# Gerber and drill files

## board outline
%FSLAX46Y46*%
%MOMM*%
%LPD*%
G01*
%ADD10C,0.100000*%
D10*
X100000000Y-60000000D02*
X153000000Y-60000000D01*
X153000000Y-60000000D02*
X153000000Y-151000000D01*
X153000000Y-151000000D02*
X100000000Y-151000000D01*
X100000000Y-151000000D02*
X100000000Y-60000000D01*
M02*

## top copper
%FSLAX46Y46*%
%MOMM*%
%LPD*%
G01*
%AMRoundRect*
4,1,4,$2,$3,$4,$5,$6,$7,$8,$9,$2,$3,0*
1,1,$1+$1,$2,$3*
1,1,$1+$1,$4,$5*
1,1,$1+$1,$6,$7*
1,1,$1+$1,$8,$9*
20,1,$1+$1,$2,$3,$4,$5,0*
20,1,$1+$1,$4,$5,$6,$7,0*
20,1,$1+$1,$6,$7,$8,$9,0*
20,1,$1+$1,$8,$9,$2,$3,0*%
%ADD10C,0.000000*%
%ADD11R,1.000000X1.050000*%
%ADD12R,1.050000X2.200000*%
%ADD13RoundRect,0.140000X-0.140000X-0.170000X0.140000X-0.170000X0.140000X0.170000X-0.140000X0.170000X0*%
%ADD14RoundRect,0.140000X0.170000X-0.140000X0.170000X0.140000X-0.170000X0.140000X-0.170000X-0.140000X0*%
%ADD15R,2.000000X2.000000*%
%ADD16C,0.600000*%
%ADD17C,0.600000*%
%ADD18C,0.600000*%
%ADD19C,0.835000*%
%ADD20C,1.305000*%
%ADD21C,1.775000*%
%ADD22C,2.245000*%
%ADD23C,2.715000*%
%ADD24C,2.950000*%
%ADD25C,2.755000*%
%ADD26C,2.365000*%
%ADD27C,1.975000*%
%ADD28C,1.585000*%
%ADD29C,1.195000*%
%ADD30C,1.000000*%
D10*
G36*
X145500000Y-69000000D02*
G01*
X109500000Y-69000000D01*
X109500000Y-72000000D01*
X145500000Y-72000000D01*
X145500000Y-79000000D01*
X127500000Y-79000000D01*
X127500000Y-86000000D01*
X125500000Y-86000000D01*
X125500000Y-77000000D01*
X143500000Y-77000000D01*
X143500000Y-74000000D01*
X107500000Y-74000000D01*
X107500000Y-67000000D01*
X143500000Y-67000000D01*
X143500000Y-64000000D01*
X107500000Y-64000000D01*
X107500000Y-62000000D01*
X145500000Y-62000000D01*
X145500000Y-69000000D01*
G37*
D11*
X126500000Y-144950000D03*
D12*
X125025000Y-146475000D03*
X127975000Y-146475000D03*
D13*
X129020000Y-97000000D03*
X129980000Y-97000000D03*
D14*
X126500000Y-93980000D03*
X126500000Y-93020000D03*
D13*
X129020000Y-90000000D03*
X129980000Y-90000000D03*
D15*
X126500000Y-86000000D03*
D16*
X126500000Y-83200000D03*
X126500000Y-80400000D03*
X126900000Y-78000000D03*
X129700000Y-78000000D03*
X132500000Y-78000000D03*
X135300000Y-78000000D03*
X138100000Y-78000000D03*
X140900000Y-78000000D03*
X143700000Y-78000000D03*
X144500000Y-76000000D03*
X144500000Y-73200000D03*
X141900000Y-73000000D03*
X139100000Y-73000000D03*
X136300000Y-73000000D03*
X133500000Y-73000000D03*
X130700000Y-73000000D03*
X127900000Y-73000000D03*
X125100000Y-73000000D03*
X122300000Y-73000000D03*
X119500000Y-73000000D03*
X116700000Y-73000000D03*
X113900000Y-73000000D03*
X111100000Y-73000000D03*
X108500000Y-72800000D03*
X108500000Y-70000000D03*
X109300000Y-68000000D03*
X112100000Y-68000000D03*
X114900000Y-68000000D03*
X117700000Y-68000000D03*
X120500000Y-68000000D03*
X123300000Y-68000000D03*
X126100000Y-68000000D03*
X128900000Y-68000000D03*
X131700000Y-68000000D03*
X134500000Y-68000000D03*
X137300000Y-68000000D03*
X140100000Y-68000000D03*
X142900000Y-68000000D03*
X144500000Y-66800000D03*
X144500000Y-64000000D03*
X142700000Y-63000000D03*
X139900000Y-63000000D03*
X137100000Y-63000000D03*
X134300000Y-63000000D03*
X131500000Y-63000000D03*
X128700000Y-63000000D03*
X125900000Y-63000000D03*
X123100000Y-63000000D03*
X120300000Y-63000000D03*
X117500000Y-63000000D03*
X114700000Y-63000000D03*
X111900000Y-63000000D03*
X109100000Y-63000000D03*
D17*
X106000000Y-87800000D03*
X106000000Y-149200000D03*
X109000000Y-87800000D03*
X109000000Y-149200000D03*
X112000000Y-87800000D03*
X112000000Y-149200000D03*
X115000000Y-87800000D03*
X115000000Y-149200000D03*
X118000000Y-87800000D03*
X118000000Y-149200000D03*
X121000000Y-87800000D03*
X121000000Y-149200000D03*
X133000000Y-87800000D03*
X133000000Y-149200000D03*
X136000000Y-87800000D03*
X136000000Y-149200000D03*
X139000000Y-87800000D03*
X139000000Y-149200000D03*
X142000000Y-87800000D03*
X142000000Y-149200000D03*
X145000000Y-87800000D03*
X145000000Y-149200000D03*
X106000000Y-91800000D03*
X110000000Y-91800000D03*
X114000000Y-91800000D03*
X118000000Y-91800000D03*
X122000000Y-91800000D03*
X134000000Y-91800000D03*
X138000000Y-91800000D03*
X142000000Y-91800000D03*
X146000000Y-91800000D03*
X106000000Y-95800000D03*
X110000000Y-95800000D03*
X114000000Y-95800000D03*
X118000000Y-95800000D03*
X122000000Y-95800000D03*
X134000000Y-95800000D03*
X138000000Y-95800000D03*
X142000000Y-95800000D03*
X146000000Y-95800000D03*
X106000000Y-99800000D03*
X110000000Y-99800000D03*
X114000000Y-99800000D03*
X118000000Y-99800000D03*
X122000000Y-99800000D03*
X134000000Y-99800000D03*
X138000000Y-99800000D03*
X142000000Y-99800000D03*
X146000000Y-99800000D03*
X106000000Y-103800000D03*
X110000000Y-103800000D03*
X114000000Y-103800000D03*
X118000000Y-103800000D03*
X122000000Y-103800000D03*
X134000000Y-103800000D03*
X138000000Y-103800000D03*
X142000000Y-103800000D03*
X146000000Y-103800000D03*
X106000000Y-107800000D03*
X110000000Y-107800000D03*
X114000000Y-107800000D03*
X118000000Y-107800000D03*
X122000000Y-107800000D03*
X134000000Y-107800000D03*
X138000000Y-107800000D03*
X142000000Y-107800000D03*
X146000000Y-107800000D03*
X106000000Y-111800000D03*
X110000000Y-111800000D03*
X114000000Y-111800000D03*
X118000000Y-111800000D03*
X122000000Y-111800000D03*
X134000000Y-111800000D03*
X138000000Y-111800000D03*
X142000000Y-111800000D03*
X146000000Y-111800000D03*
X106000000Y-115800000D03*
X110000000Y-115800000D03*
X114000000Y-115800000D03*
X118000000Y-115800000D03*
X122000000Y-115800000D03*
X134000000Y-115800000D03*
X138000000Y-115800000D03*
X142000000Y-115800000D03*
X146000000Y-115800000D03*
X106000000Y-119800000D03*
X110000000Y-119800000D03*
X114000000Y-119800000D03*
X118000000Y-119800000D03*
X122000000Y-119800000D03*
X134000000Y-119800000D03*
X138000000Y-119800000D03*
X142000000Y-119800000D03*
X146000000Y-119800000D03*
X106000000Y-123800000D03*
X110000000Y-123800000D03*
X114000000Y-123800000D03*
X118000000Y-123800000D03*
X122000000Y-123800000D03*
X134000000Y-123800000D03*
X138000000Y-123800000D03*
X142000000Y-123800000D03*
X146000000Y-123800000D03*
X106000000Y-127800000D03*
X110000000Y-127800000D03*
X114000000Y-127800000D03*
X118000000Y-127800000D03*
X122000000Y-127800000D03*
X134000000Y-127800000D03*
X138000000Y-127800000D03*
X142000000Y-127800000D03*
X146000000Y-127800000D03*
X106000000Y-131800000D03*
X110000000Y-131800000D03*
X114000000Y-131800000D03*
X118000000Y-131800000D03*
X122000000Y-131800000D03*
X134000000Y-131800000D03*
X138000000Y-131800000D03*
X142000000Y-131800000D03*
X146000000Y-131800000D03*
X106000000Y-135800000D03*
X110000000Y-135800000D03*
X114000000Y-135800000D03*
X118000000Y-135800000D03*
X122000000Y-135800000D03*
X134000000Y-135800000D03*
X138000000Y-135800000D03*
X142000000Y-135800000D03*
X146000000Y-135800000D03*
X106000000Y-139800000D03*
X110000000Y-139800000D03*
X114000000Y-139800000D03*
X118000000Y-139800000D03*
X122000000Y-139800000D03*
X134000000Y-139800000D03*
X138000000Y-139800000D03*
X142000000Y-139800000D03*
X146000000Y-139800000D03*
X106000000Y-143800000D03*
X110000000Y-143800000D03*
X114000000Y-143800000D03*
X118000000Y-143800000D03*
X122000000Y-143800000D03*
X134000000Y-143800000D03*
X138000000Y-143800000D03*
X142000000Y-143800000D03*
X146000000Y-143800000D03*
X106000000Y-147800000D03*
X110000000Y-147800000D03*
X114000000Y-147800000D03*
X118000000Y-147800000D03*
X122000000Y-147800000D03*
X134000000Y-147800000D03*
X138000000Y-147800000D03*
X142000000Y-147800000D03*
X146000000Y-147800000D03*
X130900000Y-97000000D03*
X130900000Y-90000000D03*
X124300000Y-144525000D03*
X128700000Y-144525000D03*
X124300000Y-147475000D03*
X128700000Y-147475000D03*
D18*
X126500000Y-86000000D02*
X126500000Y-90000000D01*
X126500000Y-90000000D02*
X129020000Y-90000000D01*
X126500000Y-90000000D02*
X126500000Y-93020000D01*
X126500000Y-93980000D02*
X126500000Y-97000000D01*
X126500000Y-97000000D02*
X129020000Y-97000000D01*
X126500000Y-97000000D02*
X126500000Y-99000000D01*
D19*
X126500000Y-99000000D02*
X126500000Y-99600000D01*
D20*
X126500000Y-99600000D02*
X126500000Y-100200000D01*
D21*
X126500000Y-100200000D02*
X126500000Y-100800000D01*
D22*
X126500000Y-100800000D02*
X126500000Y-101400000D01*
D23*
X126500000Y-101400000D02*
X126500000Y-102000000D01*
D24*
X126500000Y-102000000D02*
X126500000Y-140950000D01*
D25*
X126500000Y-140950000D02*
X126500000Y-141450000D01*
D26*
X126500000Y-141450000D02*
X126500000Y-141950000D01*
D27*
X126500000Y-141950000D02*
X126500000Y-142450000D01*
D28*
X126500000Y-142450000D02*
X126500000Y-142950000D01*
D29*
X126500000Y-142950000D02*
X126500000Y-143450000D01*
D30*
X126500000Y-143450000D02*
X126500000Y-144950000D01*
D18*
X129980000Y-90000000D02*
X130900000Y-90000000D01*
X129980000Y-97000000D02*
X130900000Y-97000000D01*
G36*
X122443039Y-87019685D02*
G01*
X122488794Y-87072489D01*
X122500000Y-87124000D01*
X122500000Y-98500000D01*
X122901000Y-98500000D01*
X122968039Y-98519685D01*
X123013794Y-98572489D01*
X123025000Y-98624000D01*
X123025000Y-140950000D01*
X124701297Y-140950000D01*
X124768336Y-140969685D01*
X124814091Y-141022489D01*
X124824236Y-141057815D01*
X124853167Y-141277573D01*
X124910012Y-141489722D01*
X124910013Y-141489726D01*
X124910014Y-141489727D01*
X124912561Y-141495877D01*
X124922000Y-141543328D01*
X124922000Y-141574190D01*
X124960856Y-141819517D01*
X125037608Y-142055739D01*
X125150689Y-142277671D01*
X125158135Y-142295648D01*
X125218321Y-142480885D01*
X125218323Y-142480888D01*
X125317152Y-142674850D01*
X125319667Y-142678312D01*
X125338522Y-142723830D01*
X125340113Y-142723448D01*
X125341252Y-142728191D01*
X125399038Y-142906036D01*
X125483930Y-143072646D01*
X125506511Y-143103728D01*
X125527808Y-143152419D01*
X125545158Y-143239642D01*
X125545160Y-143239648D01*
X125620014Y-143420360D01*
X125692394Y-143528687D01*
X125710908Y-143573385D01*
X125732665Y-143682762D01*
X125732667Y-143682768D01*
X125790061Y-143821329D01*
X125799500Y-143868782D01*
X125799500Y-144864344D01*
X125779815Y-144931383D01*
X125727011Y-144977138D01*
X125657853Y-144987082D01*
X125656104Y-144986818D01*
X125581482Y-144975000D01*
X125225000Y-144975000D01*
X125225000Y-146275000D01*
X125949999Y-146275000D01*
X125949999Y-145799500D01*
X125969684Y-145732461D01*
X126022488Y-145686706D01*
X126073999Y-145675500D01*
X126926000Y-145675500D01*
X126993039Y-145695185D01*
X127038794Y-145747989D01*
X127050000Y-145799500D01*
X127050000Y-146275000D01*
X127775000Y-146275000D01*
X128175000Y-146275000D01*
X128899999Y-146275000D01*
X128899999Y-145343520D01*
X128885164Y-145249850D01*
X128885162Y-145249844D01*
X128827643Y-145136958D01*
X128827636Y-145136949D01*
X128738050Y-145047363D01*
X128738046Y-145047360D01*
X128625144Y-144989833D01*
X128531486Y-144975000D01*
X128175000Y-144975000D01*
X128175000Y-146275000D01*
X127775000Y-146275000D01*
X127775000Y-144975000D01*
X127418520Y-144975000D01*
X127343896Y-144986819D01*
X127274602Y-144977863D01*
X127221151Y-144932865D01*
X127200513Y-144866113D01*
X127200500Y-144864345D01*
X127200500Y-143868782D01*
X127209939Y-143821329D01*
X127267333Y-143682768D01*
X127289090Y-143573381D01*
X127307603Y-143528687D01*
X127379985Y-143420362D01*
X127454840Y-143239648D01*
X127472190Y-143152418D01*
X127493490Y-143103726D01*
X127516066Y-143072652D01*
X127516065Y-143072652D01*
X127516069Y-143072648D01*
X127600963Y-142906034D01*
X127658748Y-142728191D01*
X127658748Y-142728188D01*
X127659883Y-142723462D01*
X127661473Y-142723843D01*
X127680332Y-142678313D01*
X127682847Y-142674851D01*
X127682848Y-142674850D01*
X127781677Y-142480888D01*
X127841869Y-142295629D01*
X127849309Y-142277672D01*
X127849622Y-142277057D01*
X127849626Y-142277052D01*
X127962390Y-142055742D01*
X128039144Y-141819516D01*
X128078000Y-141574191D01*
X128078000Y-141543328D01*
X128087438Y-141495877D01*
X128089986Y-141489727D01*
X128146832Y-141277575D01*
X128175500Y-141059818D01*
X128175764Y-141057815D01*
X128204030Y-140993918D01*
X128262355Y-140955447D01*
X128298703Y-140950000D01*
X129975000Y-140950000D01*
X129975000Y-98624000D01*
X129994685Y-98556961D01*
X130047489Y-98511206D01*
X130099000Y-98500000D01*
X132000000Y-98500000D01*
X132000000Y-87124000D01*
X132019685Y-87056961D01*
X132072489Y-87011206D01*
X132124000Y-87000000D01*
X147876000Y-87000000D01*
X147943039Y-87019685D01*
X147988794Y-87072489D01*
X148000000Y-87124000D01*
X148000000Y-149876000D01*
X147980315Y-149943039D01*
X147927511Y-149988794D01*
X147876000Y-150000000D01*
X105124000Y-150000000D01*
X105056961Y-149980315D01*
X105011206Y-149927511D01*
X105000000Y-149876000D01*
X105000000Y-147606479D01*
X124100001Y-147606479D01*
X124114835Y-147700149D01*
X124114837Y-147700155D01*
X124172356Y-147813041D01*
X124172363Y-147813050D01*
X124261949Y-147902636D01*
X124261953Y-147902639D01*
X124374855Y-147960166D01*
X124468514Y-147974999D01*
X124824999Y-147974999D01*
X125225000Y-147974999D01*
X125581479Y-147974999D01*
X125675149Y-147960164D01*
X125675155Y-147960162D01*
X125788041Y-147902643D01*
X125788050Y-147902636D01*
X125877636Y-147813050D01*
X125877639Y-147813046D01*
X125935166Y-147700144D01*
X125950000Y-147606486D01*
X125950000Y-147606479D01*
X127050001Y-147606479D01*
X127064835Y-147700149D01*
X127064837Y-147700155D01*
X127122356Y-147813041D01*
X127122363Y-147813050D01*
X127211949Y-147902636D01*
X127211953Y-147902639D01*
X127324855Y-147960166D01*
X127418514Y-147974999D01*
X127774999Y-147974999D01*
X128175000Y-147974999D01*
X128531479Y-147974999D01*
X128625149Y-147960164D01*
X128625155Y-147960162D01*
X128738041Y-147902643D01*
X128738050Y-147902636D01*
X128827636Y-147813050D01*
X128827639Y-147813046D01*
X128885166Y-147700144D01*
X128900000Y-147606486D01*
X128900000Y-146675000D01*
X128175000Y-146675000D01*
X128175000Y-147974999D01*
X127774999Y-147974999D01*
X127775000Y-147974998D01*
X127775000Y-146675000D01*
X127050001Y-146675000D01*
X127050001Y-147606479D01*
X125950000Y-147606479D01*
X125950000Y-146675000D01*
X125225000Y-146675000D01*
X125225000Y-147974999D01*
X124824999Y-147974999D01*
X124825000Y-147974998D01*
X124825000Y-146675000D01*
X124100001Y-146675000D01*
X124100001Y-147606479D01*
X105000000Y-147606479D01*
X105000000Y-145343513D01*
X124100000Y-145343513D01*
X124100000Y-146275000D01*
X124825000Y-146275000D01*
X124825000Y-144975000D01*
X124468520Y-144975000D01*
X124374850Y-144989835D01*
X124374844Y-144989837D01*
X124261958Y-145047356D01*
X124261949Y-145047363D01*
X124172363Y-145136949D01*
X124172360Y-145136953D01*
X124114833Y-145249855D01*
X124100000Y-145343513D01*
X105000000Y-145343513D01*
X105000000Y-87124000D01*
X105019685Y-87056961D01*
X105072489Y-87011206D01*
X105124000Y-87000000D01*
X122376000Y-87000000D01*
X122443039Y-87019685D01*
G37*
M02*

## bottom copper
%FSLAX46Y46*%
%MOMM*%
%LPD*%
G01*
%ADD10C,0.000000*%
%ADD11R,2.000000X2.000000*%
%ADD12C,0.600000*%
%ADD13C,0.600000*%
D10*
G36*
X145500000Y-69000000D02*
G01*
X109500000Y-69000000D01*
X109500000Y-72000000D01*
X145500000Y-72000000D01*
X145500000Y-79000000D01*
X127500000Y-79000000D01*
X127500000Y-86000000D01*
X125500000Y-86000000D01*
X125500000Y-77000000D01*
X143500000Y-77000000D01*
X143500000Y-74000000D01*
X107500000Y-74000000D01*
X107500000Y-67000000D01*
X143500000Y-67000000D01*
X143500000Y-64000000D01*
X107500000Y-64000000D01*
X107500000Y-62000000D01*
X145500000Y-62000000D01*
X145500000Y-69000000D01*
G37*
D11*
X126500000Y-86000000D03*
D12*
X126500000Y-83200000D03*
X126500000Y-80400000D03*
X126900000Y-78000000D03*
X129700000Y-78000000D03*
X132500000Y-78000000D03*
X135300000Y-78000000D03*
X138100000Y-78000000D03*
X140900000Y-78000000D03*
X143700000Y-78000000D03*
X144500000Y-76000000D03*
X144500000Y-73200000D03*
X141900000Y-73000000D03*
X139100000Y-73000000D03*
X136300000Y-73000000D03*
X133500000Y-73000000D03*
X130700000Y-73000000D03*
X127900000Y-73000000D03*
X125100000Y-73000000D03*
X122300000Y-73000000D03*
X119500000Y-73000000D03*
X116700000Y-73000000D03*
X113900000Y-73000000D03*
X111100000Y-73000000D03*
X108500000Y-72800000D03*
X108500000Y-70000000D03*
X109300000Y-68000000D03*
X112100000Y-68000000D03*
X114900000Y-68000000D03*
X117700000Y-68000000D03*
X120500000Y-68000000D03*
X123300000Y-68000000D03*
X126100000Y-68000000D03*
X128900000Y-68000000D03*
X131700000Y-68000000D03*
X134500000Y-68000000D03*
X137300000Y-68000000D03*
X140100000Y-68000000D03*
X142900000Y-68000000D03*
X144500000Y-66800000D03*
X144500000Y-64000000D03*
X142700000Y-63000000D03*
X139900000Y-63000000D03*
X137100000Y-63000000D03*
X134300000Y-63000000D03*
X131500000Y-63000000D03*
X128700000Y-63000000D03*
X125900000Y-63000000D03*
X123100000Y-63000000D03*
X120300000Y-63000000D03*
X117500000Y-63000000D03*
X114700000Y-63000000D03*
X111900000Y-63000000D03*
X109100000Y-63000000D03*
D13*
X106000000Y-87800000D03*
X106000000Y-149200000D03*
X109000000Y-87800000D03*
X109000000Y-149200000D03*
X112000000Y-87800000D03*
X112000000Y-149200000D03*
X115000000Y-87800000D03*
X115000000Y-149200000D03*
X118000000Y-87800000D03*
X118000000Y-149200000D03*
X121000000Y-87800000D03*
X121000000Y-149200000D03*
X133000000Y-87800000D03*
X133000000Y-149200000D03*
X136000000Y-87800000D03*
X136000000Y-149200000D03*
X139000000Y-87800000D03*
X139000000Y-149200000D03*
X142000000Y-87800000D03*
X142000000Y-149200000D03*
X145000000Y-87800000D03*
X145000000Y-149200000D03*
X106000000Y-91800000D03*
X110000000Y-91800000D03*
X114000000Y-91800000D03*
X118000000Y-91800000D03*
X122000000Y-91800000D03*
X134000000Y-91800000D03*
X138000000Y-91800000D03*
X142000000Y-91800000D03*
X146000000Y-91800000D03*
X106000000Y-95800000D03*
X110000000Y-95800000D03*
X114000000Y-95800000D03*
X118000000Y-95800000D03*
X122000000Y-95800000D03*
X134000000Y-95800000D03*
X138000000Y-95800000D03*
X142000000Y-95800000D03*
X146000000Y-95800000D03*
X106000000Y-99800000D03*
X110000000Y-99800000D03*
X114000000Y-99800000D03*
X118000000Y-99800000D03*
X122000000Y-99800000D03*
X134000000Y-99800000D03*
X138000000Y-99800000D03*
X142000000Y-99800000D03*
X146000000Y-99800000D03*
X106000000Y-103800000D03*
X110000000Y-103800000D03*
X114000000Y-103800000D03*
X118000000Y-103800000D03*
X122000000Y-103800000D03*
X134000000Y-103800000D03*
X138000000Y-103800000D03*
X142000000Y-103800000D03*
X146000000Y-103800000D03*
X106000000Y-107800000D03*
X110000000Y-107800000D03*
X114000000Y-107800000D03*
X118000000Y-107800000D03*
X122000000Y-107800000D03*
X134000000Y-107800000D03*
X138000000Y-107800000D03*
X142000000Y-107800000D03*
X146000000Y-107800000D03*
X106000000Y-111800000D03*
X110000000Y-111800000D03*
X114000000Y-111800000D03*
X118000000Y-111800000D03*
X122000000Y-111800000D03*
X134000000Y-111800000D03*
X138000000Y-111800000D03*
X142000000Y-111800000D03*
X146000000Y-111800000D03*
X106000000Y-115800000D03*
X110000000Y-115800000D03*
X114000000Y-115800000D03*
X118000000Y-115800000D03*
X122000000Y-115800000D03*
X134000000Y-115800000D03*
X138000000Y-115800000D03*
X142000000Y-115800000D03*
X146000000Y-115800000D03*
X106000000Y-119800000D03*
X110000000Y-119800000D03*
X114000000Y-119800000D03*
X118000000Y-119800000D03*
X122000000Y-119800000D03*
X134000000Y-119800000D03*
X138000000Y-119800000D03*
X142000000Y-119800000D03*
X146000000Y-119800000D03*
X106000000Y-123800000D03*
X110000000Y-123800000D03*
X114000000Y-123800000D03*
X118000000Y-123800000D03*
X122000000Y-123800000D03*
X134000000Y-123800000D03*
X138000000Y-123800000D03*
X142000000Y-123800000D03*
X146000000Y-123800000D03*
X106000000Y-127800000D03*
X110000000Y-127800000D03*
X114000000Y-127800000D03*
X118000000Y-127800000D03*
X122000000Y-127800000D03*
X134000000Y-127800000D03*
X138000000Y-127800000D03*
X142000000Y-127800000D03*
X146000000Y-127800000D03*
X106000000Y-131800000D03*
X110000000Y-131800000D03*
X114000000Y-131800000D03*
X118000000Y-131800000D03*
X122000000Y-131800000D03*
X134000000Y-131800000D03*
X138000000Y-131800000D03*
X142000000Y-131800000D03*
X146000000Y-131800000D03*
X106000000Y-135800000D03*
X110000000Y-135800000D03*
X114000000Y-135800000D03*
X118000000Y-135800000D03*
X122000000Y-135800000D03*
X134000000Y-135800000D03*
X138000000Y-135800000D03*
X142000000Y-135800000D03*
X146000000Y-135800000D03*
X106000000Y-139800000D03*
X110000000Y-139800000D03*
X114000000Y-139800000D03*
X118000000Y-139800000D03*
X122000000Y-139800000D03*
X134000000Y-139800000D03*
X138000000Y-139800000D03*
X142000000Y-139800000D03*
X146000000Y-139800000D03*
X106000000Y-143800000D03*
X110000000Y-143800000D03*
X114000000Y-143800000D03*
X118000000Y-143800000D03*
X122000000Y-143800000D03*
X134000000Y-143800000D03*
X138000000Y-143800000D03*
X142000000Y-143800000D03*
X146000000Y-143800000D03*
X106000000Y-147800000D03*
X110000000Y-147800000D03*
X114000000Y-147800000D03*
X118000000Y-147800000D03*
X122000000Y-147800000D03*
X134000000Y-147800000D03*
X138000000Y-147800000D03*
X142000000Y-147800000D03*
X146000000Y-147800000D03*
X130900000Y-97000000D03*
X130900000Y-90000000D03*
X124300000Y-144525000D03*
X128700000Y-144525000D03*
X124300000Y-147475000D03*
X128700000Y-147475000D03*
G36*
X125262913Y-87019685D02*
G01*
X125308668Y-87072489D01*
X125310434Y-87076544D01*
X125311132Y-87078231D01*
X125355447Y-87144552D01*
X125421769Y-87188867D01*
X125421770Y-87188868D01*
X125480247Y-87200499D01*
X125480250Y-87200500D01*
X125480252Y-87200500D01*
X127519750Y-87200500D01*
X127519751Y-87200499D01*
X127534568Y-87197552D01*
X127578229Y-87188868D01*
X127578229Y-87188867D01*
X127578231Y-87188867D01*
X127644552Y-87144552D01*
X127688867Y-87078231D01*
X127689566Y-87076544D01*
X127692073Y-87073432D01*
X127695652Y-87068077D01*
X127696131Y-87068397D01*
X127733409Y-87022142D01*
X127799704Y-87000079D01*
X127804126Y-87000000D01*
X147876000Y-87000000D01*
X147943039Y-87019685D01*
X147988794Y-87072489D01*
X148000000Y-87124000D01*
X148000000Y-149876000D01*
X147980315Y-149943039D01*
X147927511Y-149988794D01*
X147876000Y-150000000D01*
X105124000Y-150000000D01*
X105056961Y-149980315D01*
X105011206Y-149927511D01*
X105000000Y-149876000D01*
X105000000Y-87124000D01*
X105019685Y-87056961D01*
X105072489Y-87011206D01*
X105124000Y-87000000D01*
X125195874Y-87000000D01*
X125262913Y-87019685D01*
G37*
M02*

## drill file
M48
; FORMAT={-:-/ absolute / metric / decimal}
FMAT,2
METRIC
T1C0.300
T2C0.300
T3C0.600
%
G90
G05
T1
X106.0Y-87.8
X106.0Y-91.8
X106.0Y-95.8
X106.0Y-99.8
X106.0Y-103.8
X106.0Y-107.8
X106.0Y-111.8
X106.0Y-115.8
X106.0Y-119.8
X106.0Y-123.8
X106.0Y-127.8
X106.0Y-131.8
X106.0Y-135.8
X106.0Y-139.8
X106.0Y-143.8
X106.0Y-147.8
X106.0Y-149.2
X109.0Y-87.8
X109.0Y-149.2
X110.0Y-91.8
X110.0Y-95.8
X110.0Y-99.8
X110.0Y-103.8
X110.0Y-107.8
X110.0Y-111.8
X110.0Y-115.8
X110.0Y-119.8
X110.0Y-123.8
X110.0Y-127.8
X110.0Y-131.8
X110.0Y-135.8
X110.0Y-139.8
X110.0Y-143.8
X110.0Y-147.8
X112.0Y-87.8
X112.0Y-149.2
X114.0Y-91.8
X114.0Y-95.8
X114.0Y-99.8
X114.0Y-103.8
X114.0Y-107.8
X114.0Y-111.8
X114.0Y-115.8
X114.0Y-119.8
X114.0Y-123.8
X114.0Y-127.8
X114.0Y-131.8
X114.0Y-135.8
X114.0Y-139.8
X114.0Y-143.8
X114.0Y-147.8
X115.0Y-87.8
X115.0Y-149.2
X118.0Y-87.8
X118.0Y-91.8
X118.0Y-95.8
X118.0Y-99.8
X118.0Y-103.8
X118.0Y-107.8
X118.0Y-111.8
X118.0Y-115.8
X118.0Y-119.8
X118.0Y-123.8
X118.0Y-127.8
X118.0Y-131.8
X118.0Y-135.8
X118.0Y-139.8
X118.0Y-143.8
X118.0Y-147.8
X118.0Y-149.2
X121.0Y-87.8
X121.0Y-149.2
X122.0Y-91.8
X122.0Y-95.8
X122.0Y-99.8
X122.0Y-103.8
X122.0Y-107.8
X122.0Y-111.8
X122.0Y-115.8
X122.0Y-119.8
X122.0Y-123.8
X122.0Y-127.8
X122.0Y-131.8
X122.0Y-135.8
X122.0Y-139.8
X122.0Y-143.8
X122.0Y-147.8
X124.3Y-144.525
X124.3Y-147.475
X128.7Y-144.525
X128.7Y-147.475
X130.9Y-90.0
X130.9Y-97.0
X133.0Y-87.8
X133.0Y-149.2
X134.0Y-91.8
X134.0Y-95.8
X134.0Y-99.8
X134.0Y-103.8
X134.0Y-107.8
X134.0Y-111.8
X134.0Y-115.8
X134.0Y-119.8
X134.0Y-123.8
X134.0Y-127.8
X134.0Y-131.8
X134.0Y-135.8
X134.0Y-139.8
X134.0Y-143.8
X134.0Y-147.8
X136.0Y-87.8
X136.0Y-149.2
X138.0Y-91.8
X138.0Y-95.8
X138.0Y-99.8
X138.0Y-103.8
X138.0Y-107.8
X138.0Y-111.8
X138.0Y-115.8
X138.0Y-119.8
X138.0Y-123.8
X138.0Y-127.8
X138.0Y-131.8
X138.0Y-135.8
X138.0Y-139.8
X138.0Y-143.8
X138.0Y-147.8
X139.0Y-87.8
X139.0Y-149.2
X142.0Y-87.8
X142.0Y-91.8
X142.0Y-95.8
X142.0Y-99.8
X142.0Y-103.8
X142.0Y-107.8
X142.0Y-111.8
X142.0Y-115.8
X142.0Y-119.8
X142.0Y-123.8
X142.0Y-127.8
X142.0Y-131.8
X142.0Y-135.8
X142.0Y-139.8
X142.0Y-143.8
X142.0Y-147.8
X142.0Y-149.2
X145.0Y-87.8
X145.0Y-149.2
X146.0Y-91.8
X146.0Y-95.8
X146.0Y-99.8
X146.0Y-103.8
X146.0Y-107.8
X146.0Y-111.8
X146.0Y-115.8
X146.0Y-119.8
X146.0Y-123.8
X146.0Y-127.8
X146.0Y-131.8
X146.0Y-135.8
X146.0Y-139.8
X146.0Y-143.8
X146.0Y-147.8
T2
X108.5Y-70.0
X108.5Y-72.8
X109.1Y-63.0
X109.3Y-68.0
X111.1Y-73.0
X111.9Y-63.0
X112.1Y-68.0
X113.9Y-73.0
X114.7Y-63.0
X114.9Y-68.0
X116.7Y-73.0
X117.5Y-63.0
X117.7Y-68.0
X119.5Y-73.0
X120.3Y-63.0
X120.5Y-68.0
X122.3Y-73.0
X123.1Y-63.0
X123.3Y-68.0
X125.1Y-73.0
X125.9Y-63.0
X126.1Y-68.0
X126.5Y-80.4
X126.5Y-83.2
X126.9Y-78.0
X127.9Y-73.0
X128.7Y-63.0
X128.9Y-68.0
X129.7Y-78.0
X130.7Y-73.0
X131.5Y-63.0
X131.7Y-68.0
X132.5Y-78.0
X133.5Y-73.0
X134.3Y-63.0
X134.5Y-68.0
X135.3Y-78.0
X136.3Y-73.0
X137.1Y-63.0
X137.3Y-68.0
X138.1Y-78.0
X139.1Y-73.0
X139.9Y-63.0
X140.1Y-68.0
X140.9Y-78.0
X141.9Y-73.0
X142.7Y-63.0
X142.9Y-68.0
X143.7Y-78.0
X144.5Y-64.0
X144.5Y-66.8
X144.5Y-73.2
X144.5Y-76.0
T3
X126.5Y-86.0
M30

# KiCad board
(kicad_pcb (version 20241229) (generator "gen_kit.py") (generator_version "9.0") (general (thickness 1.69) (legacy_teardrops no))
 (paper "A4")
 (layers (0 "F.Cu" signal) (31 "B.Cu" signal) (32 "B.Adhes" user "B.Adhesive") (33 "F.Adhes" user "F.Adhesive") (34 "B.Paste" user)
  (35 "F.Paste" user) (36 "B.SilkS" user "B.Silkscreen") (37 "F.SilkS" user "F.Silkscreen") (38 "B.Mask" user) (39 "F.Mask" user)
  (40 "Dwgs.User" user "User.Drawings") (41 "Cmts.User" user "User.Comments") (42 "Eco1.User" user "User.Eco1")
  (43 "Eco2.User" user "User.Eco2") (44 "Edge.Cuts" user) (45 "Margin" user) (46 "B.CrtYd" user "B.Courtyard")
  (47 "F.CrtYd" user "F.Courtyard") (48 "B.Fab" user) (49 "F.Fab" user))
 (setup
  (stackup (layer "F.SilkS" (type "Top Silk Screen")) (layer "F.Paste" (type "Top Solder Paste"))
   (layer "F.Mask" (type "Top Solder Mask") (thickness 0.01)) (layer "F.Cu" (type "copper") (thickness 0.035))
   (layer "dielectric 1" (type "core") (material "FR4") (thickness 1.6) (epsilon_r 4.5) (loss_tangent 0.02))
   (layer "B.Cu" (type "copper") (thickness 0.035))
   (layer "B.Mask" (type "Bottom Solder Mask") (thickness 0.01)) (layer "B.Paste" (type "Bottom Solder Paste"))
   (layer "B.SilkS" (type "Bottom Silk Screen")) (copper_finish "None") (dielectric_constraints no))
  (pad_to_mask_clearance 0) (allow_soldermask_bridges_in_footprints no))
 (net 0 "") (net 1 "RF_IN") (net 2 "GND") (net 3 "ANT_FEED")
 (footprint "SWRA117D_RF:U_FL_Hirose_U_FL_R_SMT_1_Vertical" (layer "F.Cu") (at 126.5 146 270)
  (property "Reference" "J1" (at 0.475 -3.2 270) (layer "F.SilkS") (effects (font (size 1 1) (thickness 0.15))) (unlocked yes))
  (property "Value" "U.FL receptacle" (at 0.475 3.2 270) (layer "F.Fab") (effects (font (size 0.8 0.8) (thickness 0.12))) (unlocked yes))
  (pad "1" smd rect (at -1.05 0 270) (size 1.05 1) (layers "F.Cu" "F.Paste" "F.Mask") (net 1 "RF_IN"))
  (pad "2" smd rect (at 0.475 1.475 270) (size 2.2 1.05) (layers "F.Cu" "F.Paste" "F.Mask") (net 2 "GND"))
  (pad "2" smd rect (at 0.475 -1.475 270) (size 2.2 1.05) (layers "F.Cu" "F.Paste" "F.Mask") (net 2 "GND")))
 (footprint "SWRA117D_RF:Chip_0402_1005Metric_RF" (layer "F.Cu") (at 129.5 97)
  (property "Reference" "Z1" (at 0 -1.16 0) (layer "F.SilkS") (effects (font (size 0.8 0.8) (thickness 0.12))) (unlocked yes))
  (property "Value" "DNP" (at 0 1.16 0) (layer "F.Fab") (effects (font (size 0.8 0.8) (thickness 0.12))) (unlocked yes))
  (pad "1" smd roundrect (at -0.48 0) (size 0.56 0.62) (layers "F.Cu" "F.Paste" "F.Mask") (roundrect_rratio 0.25) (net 1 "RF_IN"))
  (pad "2" smd roundrect (at 0.48 0) (size 0.56 0.62) (layers "F.Cu" "F.Paste" "F.Mask") (roundrect_rratio 0.25) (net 2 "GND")))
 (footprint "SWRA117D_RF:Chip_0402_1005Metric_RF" (layer "F.Cu") (at 126.5 93.5 90)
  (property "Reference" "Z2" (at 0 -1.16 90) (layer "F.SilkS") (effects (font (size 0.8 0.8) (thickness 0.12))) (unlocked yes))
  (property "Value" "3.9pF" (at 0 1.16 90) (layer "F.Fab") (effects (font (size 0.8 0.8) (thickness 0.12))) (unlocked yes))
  (pad "1" smd roundrect (at -0.48 0 90) (size 0.56 0.62) (layers "F.Cu" "F.Paste" "F.Mask") (roundrect_rratio 0.25) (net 1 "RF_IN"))
  (pad "2" smd roundrect (at 0.48 0 90) (size 0.56 0.62) (layers "F.Cu" "F.Paste" "F.Mask") (roundrect_rratio 0.25) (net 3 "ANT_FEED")))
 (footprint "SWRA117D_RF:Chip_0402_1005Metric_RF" (layer "F.Cu") (at 129.5 90)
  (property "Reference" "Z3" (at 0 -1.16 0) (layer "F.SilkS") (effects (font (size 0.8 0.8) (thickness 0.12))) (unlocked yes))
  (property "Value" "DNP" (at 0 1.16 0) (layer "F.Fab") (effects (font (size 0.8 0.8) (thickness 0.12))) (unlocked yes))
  (pad "1" smd roundrect (at -0.48 0) (size 0.56 0.62) (layers "F.Cu" "F.Paste" "F.Mask") (roundrect_rratio 0.25) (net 3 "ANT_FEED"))
  (pad "2" smd roundrect (at 0.48 0) (size 0.56 0.62) (layers "F.Cu" "F.Paste" "F.Mask") (roundrect_rratio 0.25) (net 2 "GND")))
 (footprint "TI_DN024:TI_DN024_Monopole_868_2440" (layer "F.Cu") (at 126.5 86)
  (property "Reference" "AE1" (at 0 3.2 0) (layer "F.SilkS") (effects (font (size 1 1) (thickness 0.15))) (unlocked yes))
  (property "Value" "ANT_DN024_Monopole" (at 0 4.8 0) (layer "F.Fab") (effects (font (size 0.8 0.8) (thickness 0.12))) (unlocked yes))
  (fp_poly
   (pts (xy 1 0) (xy 1 -7) (xy 19 -7) (xy 19 -14) (xy -17 -14) (xy -17 -17) (xy 19 -17) (xy 19 -24) (xy -19 -24) (xy -19 -22) (xy 17 -22)
    (xy 17 -19) (xy -19 -19) (xy -19 -12) (xy 17 -12) (xy 17 -9) (xy -1 -9) (xy -1 0))
   (stroke (width 0) (type solid)) (fill yes) (layer "F.Cu"))
  (fp_poly
   (pts (xy 1 0) (xy 1 -7) (xy 19 -7) (xy 19 -14) (xy -17 -14) (xy -17 -17) (xy 19 -17) (xy 19 -24) (xy -19 -24) (xy -19 -22) (xy 17 -22)
    (xy 17 -19) (xy -19 -19) (xy -19 -12) (xy 17 -12) (xy 17 -9) (xy -1 -9) (xy -1 0))
   (stroke (width 0) (type solid)) (fill yes) (layer "B.Cu"))
  (pad "1" thru_hole rect (at 0 0) (size 2 2) (drill 0.6) (layers "*.Cu" "*.Mask") (remove_unused_layers no) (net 3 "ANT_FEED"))
  (pad "1" thru_hole circle (at 0 -2.8) (size 0.6 0.6) (drill 0.3) (layers "*.Cu") (remove_unused_layers no) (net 3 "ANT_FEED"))
  (pad "1" thru_hole circle (at 0 -5.6) (size 0.6 0.6) (drill 0.3) (layers "*.Cu") (remove_unused_layers no) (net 3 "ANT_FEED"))
  (pad "1" thru_hole circle (at 0.4 -8) (size 0.6 0.6) (drill 0.3) (layers "*.Cu") (remove_unused_layers no) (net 3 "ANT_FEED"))
  (pad "1" thru_hole circle (at 3.2 -8) (size 0.6 0.6) (drill 0.3) (layers "*.Cu") (remove_unused_layers no) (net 3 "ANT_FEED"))
  (pad "1" thru_hole circle (at 6 -8) (size 0.6 0.6) (drill 0.3) (layers "*.Cu") (remove_unused_layers no) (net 3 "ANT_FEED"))
  (pad "1" thru_hole circle (at 8.8 -8) (size 0.6 0.6) (drill 0.3) (layers "*.Cu") (remove_unused_layers no) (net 3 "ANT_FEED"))
  (pad "1" thru_hole circle (at 11.6 -8) (size 0.6 0.6) (drill 0.3) (layers "*.Cu") (remove_unused_layers no) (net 3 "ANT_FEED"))
  (pad "1" thru_hole circle (at 14.4 -8) (size 0.6 0.6) (drill 0.3) (layers "*.Cu") (remove_unused_layers no) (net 3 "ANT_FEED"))
  (pad "1" thru_hole circle (at 17.2 -8) (size 0.6 0.6) (drill 0.3) (layers "*.Cu") (remove_unused_layers no) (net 3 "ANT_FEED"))
  (pad "1" thru_hole circle (at 18 -10) (size 0.6 0.6) (drill 0.3) (layers "*.Cu") (remove_unused_layers no) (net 3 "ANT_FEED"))
  (pad "1" thru_hole circle (at 18 -12.8) (size 0.6 0.6) (drill 0.3) (layers "*.Cu") (remove_unused_layers no) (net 3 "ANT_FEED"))
  (pad "1" thru_hole circle (at 15.4 -13) (size 0.6 0.6) (drill 0.3) (layers "*.Cu") (remove_unused_layers no) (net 3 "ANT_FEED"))
  (pad "1" thru_hole circle (at 12.6 -13) (size 0.6 0.6) (drill 0.3) (layers "*.Cu") (remove_unused_layers no) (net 3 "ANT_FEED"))
  (pad "1" thru_hole circle (at 9.8 -13) (size 0.6 0.6) (drill 0.3) (layers "*.Cu") (remove_unused_layers no) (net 3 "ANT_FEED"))
  (pad "1" thru_hole circle (at 7 -13) (size 0.6 0.6) (drill 0.3) (layers "*.Cu") (remove_unused_layers no) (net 3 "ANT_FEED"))
  (pad "1" thru_hole circle (at 4.2 -13) (size 0.6 0.6) (drill 0.3) (layers "*.Cu") (remove_unused_layers no) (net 3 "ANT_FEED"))
  (pad "1" thru_hole circle (at 1.4 -13) (size 0.6 0.6) (drill 0.3) (layers "*.Cu") (remove_unused_layers no) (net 3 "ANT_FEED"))
  (pad "1" thru_hole circle (at -1.4 -13) (size 0.6 0.6) (drill 0.3) (layers "*.Cu") (remove_unused_layers no) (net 3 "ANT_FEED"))
  (pad "1" thru_hole circle (at -4.2 -13) (size 0.6 0.6) (drill 0.3) (layers "*.Cu") (remove_unused_layers no) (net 3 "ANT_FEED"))
  (pad "1" thru_hole circle (at -7 -13) (size 0.6 0.6) (drill 0.3) (layers "*.Cu") (remove_unused_layers no) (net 3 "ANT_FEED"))
  (pad "1" thru_hole circle (at -9.8 -13) (size 0.6 0.6) (drill 0.3) (layers "*.Cu") (remove_unused_layers no) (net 3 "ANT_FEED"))
  (pad "1" thru_hole circle (at -12.6 -13) (size 0.6 0.6) (drill 0.3) (layers "*.Cu") (remove_unused_layers no) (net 3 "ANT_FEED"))
  (pad "1" thru_hole circle (at -15.4 -13) (size 0.6 0.6) (drill 0.3) (layers "*.Cu") (remove_unused_layers no) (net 3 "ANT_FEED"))
  (pad "1" thru_hole circle (at -18 -13.2) (size 0.6 0.6) (drill 0.3) (layers "*.Cu") (remove_unused_layers no) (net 3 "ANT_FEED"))
  (pad "1" thru_hole circle (at -18 -16) (size 0.6 0.6) (drill 0.3) (layers "*.Cu") (remove_unused_layers no) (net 3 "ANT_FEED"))
  (pad "1" thru_hole circle (at -17.2 -18) (size 0.6 0.6) (drill 0.3) (layers "*.Cu") (remove_unused_layers no) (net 3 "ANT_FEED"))
  (pad "1" thru_hole circle (at -14.4 -18) (size 0.6 0.6) (drill 0.3) (layers "*.Cu") (remove_unused_layers no) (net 3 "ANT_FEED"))
  (pad "1" thru_hole circle (at -11.6 -18) (size 0.6 0.6) (drill 0.3) (layers "*.Cu") (remove_unused_layers no) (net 3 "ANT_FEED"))
  (pad "1" thru_hole circle (at -8.8 -18) (size 0.6 0.6) (drill 0.3) (layers "*.Cu") (remove_unused_layers no) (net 3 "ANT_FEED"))
  (pad "1" thru_hole circle (at -6 -18) (size 0.6 0.6) (drill 0.3) (layers "*.Cu") (remove_unused_layers no) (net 3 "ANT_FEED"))
  (pad "1" thru_hole circle (at -3.2 -18) (size 0.6 0.6) (drill 0.3) (layers "*.Cu") (remove_unused_layers no) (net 3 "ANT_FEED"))
  (pad "1" thru_hole circle (at -0.4 -18) (size 0.6 0.6) (drill 0.3) (layers "*.Cu") (remove_unused_layers no) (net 3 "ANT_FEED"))
  (pad "1" thru_hole circle (at 2.4 -18) (size 0.6 0.6) (drill 0.3) (layers "*.Cu") (remove_unused_layers no) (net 3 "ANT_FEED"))
  (pad "1" thru_hole circle (at 5.2 -18) (size 0.6 0.6) (drill 0.3) (layers "*.Cu") (remove_unused_layers no) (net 3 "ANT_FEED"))
  (pad "1" thru_hole circle (at 8 -18) (size 0.6 0.6) (drill 0.3) (layers "*.Cu") (remove_unused_layers no) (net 3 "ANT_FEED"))
  (pad "1" thru_hole circle (at 10.8 -18) (size 0.6 0.6) (drill 0.3) (layers "*.Cu") (remove_unused_layers no) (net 3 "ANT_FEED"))
  (pad "1" thru_hole circle (at 13.6 -18) (size 0.6 0.6) (drill 0.3) (layers "*.Cu") (remove_unused_layers no) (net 3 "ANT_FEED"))
  (pad "1" thru_hole circle (at 16.4 -18) (size 0.6 0.6) (drill 0.3) (layers "*.Cu") (remove_unused_layers no) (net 3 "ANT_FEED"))
  (pad "1" thru_hole circle (at 18 -19.2) (size 0.6 0.6) (drill 0.3) (layers "*.Cu") (remove_unused_layers no) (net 3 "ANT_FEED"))
  (pad "1" thru_hole circle (at 18 -22) (size 0.6 0.6) (drill 0.3) (layers "*.Cu") (remove_unused_layers no) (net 3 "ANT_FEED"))
  (pad "1" thru_hole circle (at 16.2 -23) (size 0.6 0.6) (drill 0.3) (layers "*.Cu") (remove_unused_layers no) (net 3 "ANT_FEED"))
  (pad "1" thru_hole circle (at 13.4 -23) (size 0.6 0.6) (drill 0.3) (layers "*.Cu") (remove_unused_layers no) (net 3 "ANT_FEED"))
  (pad "1" thru_hole circle (at 10.6 -23) (size 0.6 0.6) (drill 0.3) (layers "*.Cu") (remove_unused_layers no) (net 3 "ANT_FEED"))
  (pad "1" thru_hole circle (at 7.8 -23) (size 0.6 0.6) (drill 0.3) (layers "*.Cu") (remove_unused_layers no) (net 3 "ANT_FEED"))
  (pad "1" thru_hole circle (at 5 -23) (size 0.6 0.6) (drill 0.3) (layers "*.Cu") (remove_unused_layers no) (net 3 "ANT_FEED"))
  (pad "1" thru_hole circle (at 2.2 -23) (size 0.6 0.6) (drill 0.3) (layers "*.Cu") (remove_unused_layers no) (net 3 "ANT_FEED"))
  (pad "1" thru_hole circle (at -0.6 -23) (size 0.6 0.6) (drill 0.3) (layers "*.Cu") (remove_unused_layers no) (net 3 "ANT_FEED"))
  (pad "1" thru_hole circle (at -3.4 -23) (size 0.6 0.6) (drill 0.3) (layers "*.Cu") (remove_unused_layers no) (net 3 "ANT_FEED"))
  (pad "1" thru_hole circle (at -6.2 -23) (size 0.6 0.6) (drill 0.3) (layers "*.Cu") (remove_unused_layers no) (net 3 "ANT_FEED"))
  (pad "1" thru_hole circle (at -9 -23) (size 0.6 0.6) (drill 0.3) (layers "*.Cu") (remove_unused_layers no) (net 3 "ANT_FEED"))
  (pad "1" thru_hole circle (at -11.8 -23) (size 0.6 0.6) (drill 0.3) (layers "*.Cu") (remove_unused_layers no) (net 3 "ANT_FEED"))
  (pad "1" thru_hole circle (at -14.6 -23) (size 0.6 0.6) (drill 0.3) (layers "*.Cu") (remove_unused_layers no) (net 3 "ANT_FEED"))
  (pad "1" thru_hole circle (at -17.4 -23) (size 0.6 0.6) (drill 0.3) (layers "*.Cu") (remove_unused_layers no) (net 3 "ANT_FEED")))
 (gr_line (start 100 60) (end 153 60) (stroke (width 0.1) (type solid)) (layer "Edge.Cuts"))
 (gr_line (start 153 60) (end 153 151) (stroke (width 0.1) (type solid)) (layer "Edge.Cuts"))
 (gr_line (start 153 151) (end 100 151) (stroke (width 0.1) (type solid)) (layer "Edge.Cuts"))
 (gr_line (start 100 151) (end 100 60) (stroke (width 0.1) (type solid)) (layer "Edge.Cuts"))
 (segment (start 126.5 86) (end 126.5 90) (width 0.6) (layer "F.Cu") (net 3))
 (segment (start 126.5 90) (end 129.02 90) (width 0.6) (layer "F.Cu") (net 3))
 (segment (start 126.5 90) (end 126.5 93.02) (width 0.6) (layer "F.Cu") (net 3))
 (segment (start 126.5 93.98) (end 126.5 97) (width 0.6) (layer "F.Cu") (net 1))
 (segment (start 126.5 97) (end 129.02 97) (width 0.6) (layer "F.Cu") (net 1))
 (segment (start 126.5 97) (end 126.5 99) (width 0.6) (layer "F.Cu") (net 1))
 (segment (start 126.5 99) (end 126.5 99.6) (width 0.835) (layer "F.Cu") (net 1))
 (segment (start 126.5 99.6) (end 126.5 100.2) (width 1.305) (layer "F.Cu") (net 1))
 (segment (start 126.5 100.2) (end 126.5 100.8) (width 1.775) (layer "F.Cu") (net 1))
 (segment (start 126.5 100.8) (end 126.5 101.4) (width 2.245) (layer "F.Cu") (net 1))
 (segment (start 126.5 101.4) (end 126.5 102) (width 2.715) (layer "F.Cu") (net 1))
 (segment (start 126.5 102) (end 126.5 140.95) (width 2.95) (layer "F.Cu") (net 1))
 (segment (start 126.5 140.95) (end 126.5 141.45) (width 2.755) (layer "F.Cu") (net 1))
 (segment (start 126.5 141.45) (end 126.5 141.95) (width 2.365) (layer "F.Cu") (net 1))
 (segment (start 126.5 141.95) (end 126.5 142.45) (width 1.975) (layer "F.Cu") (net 1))
 (segment (start 126.5 142.45) (end 126.5 142.95) (width 1.585) (layer "F.Cu") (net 1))
 (segment (start 126.5 142.95) (end 126.5 143.45) (width 1.195) (layer "F.Cu") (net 1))
 (segment (start 126.5 143.45) (end 126.5 144.95) (width 1) (layer "F.Cu") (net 1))
 (segment (start 129.98 90) (end 130.9 90) (width 0.6) (layer "F.Cu") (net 2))
 (segment (start 129.98 97) (end 130.9 97) (width 0.6) (layer "F.Cu") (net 2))
 (via (at 106 87.8) (size 0.6) (drill 0.3) (layers "F.Cu" "B.Cu") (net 2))
 (via (at 106 149.2) (size 0.6) (drill 0.3) (layers "F.Cu" "B.Cu") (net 2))
 (via (at 109 87.8) (size 0.6) (drill 0.3) (layers "F.Cu" "B.Cu") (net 2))
 (via (at 109 149.2) (size 0.6) (drill 0.3) (layers "F.Cu" "B.Cu") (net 2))
 (via (at 112 87.8) (size 0.6) (drill 0.3) (layers "F.Cu" "B.Cu") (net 2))
 (via (at 112 149.2) (size 0.6) (drill 0.3) (layers "F.Cu" "B.Cu") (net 2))
 (via (at 115 87.8) (size 0.6) (drill 0.3) (layers "F.Cu" "B.Cu") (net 2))
 (via (at 115 149.2) (size 0.6) (drill 0.3) (layers "F.Cu" "B.Cu") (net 2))
 (via (at 118 87.8) (size 0.6) (drill 0.3) (layers "F.Cu" "B.Cu") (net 2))
 (via (at 118 149.2) (size 0.6) (drill 0.3) (layers "F.Cu" "B.Cu") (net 2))
 (via (at 121 87.8) (size 0.6) (drill 0.3) (layers "F.Cu" "B.Cu") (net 2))
 (via (at 121 149.2) (size 0.6) (drill 0.3) (layers "F.Cu" "B.Cu") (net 2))
 (via (at 133 87.8) (size 0.6) (drill 0.3) (layers "F.Cu" "B.Cu") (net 2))
 (via (at 133 149.2) (size 0.6) (drill 0.3) (layers "F.Cu" "B.Cu") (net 2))
 (via (at 136 87.8) (size 0.6) (drill 0.3) (layers "F.Cu" "B.Cu") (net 2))
 (via (at 136 149.2) (size 0.6) (drill 0.3) (layers "F.Cu" "B.Cu") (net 2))
 (via (at 139 87.8) (size 0.6) (drill 0.3) (layers "F.Cu" "B.Cu") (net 2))
 (via (at 139 149.2) (size 0.6) (drill 0.3) (layers "F.Cu" "B.Cu") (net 2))
 (via (at 142 87.8) (size 0.6) (drill 0.3) (layers "F.Cu" "B.Cu") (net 2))
 (via (at 142 149.2) (size 0.6) (drill 0.3) (layers "F.Cu" "B.Cu") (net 2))
 (via (at 145 87.8) (size 0.6) (drill 0.3) (layers "F.Cu" "B.Cu") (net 2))
 (via (at 145 149.2) (size 0.6) (drill 0.3) (layers "F.Cu" "B.Cu") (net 2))
 (via (at 106 91.8) (size 0.6) (drill 0.3) (layers "F.Cu" "B.Cu") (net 2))
 (via (at 110 91.8) (size 0.6) (drill 0.3) (layers "F.Cu" "B.Cu") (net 2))
 (via (at 114 91.8) (size 0.6) (drill 0.3) (layers "F.Cu" "B.Cu") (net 2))
 (via (at 118 91.8) (size 0.6) (drill 0.3) (layers "F.Cu" "B.Cu") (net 2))
 (via (at 122 91.8) (size 0.6) (drill 0.3) (layers "F.Cu" "B.Cu") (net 2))
 (via (at 134 91.8) (size 0.6) (drill 0.3) (layers "F.Cu" "B.Cu") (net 2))
 (via (at 138 91.8) (size 0.6) (drill 0.3) (layers "F.Cu" "B.Cu") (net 2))
 (via (at 142 91.8) (size 0.6) (drill 0.3) (layers "F.Cu" "B.Cu") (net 2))
 (via (at 146 91.8) (size 0.6) (drill 0.3) (layers "F.Cu" "B.Cu") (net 2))
 (via (at 106 95.8) (size 0.6) (drill 0.3) (layers "F.Cu" "B.Cu") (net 2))
 (via (at 110 95.8) (size 0.6) (drill 0.3) (layers "F.Cu" "B.Cu") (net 2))
 (via (at 114 95.8) (size 0.6) (drill 0.3) (layers "F.Cu" "B.Cu") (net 2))
 (via (at 118 95.8) (size 0.6) (drill 0.3) (layers "F.Cu" "B.Cu") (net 2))
 (via (at 122 95.8) (size 0.6) (drill 0.3) (layers "F.Cu" "B.Cu") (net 2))
 (via (at 134 95.8) (size 0.6) (drill 0.3) (layers "F.Cu" "B.Cu") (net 2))
 (via (at 138 95.8) (size 0.6) (drill 0.3) (layers "F.Cu" "B.Cu") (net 2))
 (via (at 142 95.8) (size 0.6) (drill 0.3) (layers "F.Cu" "B.Cu") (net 2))
 (via (at 146 95.8) (size 0.6) (drill 0.3) (layers "F.Cu" "B.Cu") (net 2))
 (via (at 106 99.8) (size 0.6) (drill 0.3) (layers "F.Cu" "B.Cu") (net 2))
 (via (at 110 99.8) (size 0.6) (drill 0.3) (layers "F.Cu" "B.Cu") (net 2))
 (via (at 114 99.8) (size 0.6) (drill 0.3) (layers "F.Cu" "B.Cu") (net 2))
 (via (at 118 99.8) (size 0.6) (drill 0.3) (layers "F.Cu" "B.Cu") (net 2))
 (via (at 122 99.8) (size 0.6) (drill 0.3) (layers "F.Cu" "B.Cu") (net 2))
 (via (at 134 99.8) (size 0.6) (drill 0.3) (layers "F.Cu" "B.Cu") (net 2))
 (via (at 138 99.8) (size 0.6) (drill 0.3) (layers "F.Cu" "B.Cu") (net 2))
 (via (at 142 99.8) (size 0.6) (drill 0.3) (layers "F.Cu" "B.Cu") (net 2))
 (via (at 146 99.8) (size 0.6) (drill 0.3) (layers "F.Cu" "B.Cu") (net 2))
 (via (at 106 103.8) (size 0.6) (drill 0.3) (layers "F.Cu" "B.Cu") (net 2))
 (via (at 110 103.8) (size 0.6) (drill 0.3) (layers "F.Cu" "B.Cu") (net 2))
 (via (at 114 103.8) (size 0.6) (drill 0.3) (layers "F.Cu" "B.Cu") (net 2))
 (via (at 118 103.8) (size 0.6) (drill 0.3) (layers "F.Cu" "B.Cu") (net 2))
 (via (at 122 103.8) (size 0.6) (drill 0.3) (layers "F.Cu" "B.Cu") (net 2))
 (via (at 134 103.8) (size 0.6) (drill 0.3) (layers "F.Cu" "B.Cu") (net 2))
 (via (at 138 103.8) (size 0.6) (drill 0.3) (layers "F.Cu" "B.Cu") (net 2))
 (via (at 142 103.8) (size 0.6) (drill 0.3) (layers "F.Cu" "B.Cu") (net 2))
 (via (at 146 103.8) (size 0.6) (drill 0.3) (layers "F.Cu" "B.Cu") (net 2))
 (via (at 106 107.8) (size 0.6) (drill 0.3) (layers "F.Cu" "B.Cu") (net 2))
 (via (at 110 107.8) (size 0.6) (drill 0.3) (layers "F.Cu" "B.Cu") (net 2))
 (via (at 114 107.8) (size 0.6) (drill 0.3) (layers "F.Cu" "B.Cu") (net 2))
 (via (at 118 107.8) (size 0.6) (drill 0.3) (layers "F.Cu" "B.Cu") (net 2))
 (via (at 122 107.8) (size 0.6) (drill 0.3) (layers "F.Cu" "B.Cu") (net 2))
 (via (at 134 107.8) (size 0.6) (drill 0.3) (layers "F.Cu" "B.Cu") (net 2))
 (via (at 138 107.8) (size 0.6) (drill 0.3) (layers "F.Cu" "B.Cu") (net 2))
 (via (at 142 107.8) (size 0.6) (drill 0.3) (layers "F.Cu" "B.Cu") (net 2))
 (via (at 146 107.8) (size 0.6) (drill 0.3) (layers "F.Cu" "B.Cu") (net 2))
 (via (at 106 111.8) (size 0.6) (drill 0.3) (layers "F.Cu" "B.Cu") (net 2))
 (via (at 110 111.8) (size 0.6) (drill 0.3) (layers "F.Cu" "B.Cu") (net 2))
 (via (at 114 111.8) (size 0.6) (drill 0.3) (layers "F.Cu" "B.Cu") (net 2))
 (via (at 118 111.8) (size 0.6) (drill 0.3) (layers "F.Cu" "B.Cu") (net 2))
 (via (at 122 111.8) (size 0.6) (drill 0.3) (layers "F.Cu" "B.Cu") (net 2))
 (via (at 134 111.8) (size 0.6) (drill 0.3) (layers "F.Cu" "B.Cu") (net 2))
 (via (at 138 111.8) (size 0.6) (drill 0.3) (layers "F.Cu" "B.Cu") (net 2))
 (via (at 142 111.8) (size 0.6) (drill 0.3) (layers "F.Cu" "B.Cu") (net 2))
 (via (at 146 111.8) (size 0.6) (drill 0.3) (layers "F.Cu" "B.Cu") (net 2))
 (via (at 106 115.8) (size 0.6) (drill 0.3) (layers "F.Cu" "B.Cu") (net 2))
 (via (at 110 115.8) (size 0.6) (drill 0.3) (layers "F.Cu" "B.Cu") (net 2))
 (via (at 114 115.8) (size 0.6) (drill 0.3) (layers "F.Cu" "B.Cu") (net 2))
 (via (at 118 115.8) (size 0.6) (drill 0.3) (layers "F.Cu" "B.Cu") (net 2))
 (via (at 122 115.8) (size 0.6) (drill 0.3) (layers "F.Cu" "B.Cu") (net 2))
 (via (at 134 115.8) (size 0.6) (drill 0.3) (layers "F.Cu" "B.Cu") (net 2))
 (via (at 138 115.8) (size 0.6) (drill 0.3) (layers "F.Cu" "B.Cu") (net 2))
 (via (at 142 115.8) (size 0.6) (drill 0.3) (layers "F.Cu" "B.Cu") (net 2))
 (via (at 146 115.8) (size 0.6) (drill 0.3) (layers "F.Cu" "B.Cu") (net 2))
 (via (at 106 119.8) (size 0.6) (drill 0.3) (layers "F.Cu" "B.Cu") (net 2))
 (via (at 110 119.8) (size 0.6) (drill 0.3) (layers "F.Cu" "B.Cu") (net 2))
 (via (at 114 119.8) (size 0.6) (drill 0.3) (layers "F.Cu" "B.Cu") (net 2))
 (via (at 118 119.8) (size 0.6) (drill 0.3) (layers "F.Cu" "B.Cu") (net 2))
 (via (at 122 119.8) (size 0.6) (drill 0.3) (layers "F.Cu" "B.Cu") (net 2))
 (via (at 134 119.8) (size 0.6) (drill 0.3) (layers "F.Cu" "B.Cu") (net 2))
 (via (at 138 119.8) (size 0.6) (drill 0.3) (layers "F.Cu" "B.Cu") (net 2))
 (via (at 142 119.8) (size 0.6) (drill 0.3) (layers "F.Cu" "B.Cu") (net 2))
 (via (at 146 119.8) (size 0.6) (drill 0.3) (layers "F.Cu" "B.Cu") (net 2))
 (via (at 106 123.8) (size 0.6) (drill 0.3) (layers "F.Cu" "B.Cu") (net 2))
 (via (at 110 123.8) (size 0.6) (drill 0.3) (layers "F.Cu" "B.Cu") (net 2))
 (via (at 114 123.8) (size 0.6) (drill 0.3) (layers "F.Cu" "B.Cu") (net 2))
 (via (at 118 123.8) (size 0.6) (drill 0.3) (layers "F.Cu" "B.Cu") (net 2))
 (via (at 122 123.8) (size 0.6) (drill 0.3) (layers "F.Cu" "B.Cu") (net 2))
 (via (at 134 123.8) (size 0.6) (drill 0.3) (layers "F.Cu" "B.Cu") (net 2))
 (via (at 138 123.8) (size 0.6) (drill 0.3) (layers "F.Cu" "B.Cu") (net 2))
 (via (at 142 123.8) (size 0.6) (drill 0.3) (layers "F.Cu" "B.Cu") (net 2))
 (via (at 146 123.8) (size 0.6) (drill 0.3) (layers "F.Cu" "B.Cu") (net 2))
 (via (at 106 127.8) (size 0.6) (drill 0.3) (layers "F.Cu" "B.Cu") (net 2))
 (via (at 110 127.8) (size 0.6) (drill 0.3) (layers "F.Cu" "B.Cu") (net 2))
 (via (at 114 127.8) (size 0.6) (drill 0.3) (layers "F.Cu" "B.Cu") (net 2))
 (via (at 118 127.8) (size 0.6) (drill 0.3) (layers "F.Cu" "B.Cu") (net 2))
 (via (at 122 127.8) (size 0.6) (drill 0.3) (layers "F.Cu" "B.Cu") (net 2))
 (via (at 134 127.8) (size 0.6) (drill 0.3) (layers "F.Cu" "B.Cu") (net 2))
 (via (at 138 127.8) (size 0.6) (drill 0.3) (layers "F.Cu" "B.Cu") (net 2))
 (via (at 142 127.8) (size 0.6) (drill 0.3) (layers "F.Cu" "B.Cu") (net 2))
 (via (at 146 127.8) (size 0.6) (drill 0.3) (layers "F.Cu" "B.Cu") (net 2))
 (via (at 106 131.8) (size 0.6) (drill 0.3) (layers "F.Cu" "B.Cu") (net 2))
 (via (at 110 131.8) (size 0.6) (drill 0.3) (layers "F.Cu" "B.Cu") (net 2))
 (via (at 114 131.8) (size 0.6) (drill 0.3) (layers "F.Cu" "B.Cu") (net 2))
 (via (at 118 131.8) (size 0.6) (drill 0.3) (layers "F.Cu" "B.Cu") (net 2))
 (via (at 122 131.8) (size 0.6) (drill 0.3) (layers "F.Cu" "B.Cu") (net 2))
 (via (at 134 131.8) (size 0.6) (drill 0.3) (layers "F.Cu" "B.Cu") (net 2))
 (via (at 138 131.8) (size 0.6) (drill 0.3) (layers "F.Cu" "B.Cu") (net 2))
 (via (at 142 131.8) (size 0.6) (drill 0.3) (layers "F.Cu" "B.Cu") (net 2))
 (via (at 146 131.8) (size 0.6) (drill 0.3) (layers "F.Cu" "B.Cu") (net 2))
 (via (at 106 135.8) (size 0.6) (drill 0.3) (layers "F.Cu" "B.Cu") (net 2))
 (via (at 110 135.8) (size 0.6) (drill 0.3) (layers "F.Cu" "B.Cu") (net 2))
 (via (at 114 135.8) (size 0.6) (drill 0.3) (layers "F.Cu" "B.Cu") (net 2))
 (via (at 118 135.8) (size 0.6) (drill 0.3) (layers "F.Cu" "B.Cu") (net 2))
 (via (at 122 135.8) (size 0.6) (drill 0.3) (layers "F.Cu" "B.Cu") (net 2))
 (via (at 134 135.8) (size 0.6) (drill 0.3) (layers "F.Cu" "B.Cu") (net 2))
 (via (at 138 135.8) (size 0.6) (drill 0.3) (layers "F.Cu" "B.Cu") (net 2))
 (via (at 142 135.8) (size 0.6) (drill 0.3) (layers "F.Cu" "B.Cu") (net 2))
 (via (at 146 135.8) (size 0.6) (drill 0.3) (layers "F.Cu" "B.Cu") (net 2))
 (via (at 106 139.8) (size 0.6) (drill 0.3) (layers "F.Cu" "B.Cu") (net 2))
 (via (at 110 139.8) (size 0.6) (drill 0.3) (layers "F.Cu" "B.Cu") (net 2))
 (via (at 114 139.8) (size 0.6) (drill 0.3) (layers "F.Cu" "B.Cu") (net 2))
 (via (at 118 139.8) (size 0.6) (drill 0.3) (layers "F.Cu" "B.Cu") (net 2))
 (via (at 122 139.8) (size 0.6) (drill 0.3) (layers "F.Cu" "B.Cu") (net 2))
 (via (at 134 139.8) (size 0.6) (drill 0.3) (layers "F.Cu" "B.Cu") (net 2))
 (via (at 138 139.8) (size 0.6) (drill 0.3) (layers "F.Cu" "B.Cu") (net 2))
 (via (at 142 139.8) (size 0.6) (drill 0.3) (layers "F.Cu" "B.Cu") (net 2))
 (via (at 146 139.8) (size 0.6) (drill 0.3) (layers "F.Cu" "B.Cu") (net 2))
 (via (at 106 143.8) (size 0.6) (drill 0.3) (layers "F.Cu" "B.Cu") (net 2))
 (via (at 110 143.8) (size 0.6) (drill 0.3) (layers "F.Cu" "B.Cu") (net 2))
 (via (at 114 143.8) (size 0.6) (drill 0.3) (layers "F.Cu" "B.Cu") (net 2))
 (via (at 118 143.8) (size 0.6) (drill 0.3) (layers "F.Cu" "B.Cu") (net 2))
 (via (at 122 143.8) (size 0.6) (drill 0.3) (layers "F.Cu" "B.Cu") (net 2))
 (via (at 134 143.8) (size 0.6) (drill 0.3) (layers "F.Cu" "B.Cu") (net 2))
 (via (at 138 143.8) (size 0.6) (drill 0.3) (layers "F.Cu" "B.Cu") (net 2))
 (via (at 142 143.8) (size 0.6) (drill 0.3) (layers "F.Cu" "B.Cu") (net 2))
 (via (at 146 143.8) (size 0.6) (drill 0.3) (layers "F.Cu" "B.Cu") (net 2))
 (via (at 106 147.8) (size 0.6) (drill 0.3) (layers "F.Cu" "B.Cu") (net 2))
 (via (at 110 147.8) (size 0.6) (drill 0.3) (layers "F.Cu" "B.Cu") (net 2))
 (via (at 114 147.8) (size 0.6) (drill 0.3) (layers "F.Cu" "B.Cu") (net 2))
 (via (at 118 147.8) (size 0.6) (drill 0.3) (layers "F.Cu" "B.Cu") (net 2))
 (via (at 122 147.8) (size 0.6) (drill 0.3) (layers "F.Cu" "B.Cu") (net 2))
 (via (at 134 147.8) (size 0.6) (drill 0.3) (layers "F.Cu" "B.Cu") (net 2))
 (via (at 138 147.8) (size 0.6) (drill 0.3) (layers "F.Cu" "B.Cu") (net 2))
 (via (at 142 147.8) (size 0.6) (drill 0.3) (layers "F.Cu" "B.Cu") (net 2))
 (via (at 146 147.8) (size 0.6) (drill 0.3) (layers "F.Cu" "B.Cu") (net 2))
 (via (at 130.9 97) (size 0.6) (drill 0.3) (layers "F.Cu" "B.Cu") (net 2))
 (via (at 130.9 90) (size 0.6) (drill 0.3) (layers "F.Cu" "B.Cu") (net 2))
 (via (at 124.3 144.525) (size 0.6) (drill 0.3) (layers "F.Cu" "B.Cu") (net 2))
 (via (at 128.7 144.525) (size 0.6) (drill 0.3) (layers "F.Cu" "B.Cu") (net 2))
 (via (at 124.3 147.475) (size 0.6) (drill 0.3) (layers "F.Cu" "B.Cu") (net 2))
 (via (at 128.7 147.475) (size 0.6) (drill 0.3) (layers "F.Cu" "B.Cu") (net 2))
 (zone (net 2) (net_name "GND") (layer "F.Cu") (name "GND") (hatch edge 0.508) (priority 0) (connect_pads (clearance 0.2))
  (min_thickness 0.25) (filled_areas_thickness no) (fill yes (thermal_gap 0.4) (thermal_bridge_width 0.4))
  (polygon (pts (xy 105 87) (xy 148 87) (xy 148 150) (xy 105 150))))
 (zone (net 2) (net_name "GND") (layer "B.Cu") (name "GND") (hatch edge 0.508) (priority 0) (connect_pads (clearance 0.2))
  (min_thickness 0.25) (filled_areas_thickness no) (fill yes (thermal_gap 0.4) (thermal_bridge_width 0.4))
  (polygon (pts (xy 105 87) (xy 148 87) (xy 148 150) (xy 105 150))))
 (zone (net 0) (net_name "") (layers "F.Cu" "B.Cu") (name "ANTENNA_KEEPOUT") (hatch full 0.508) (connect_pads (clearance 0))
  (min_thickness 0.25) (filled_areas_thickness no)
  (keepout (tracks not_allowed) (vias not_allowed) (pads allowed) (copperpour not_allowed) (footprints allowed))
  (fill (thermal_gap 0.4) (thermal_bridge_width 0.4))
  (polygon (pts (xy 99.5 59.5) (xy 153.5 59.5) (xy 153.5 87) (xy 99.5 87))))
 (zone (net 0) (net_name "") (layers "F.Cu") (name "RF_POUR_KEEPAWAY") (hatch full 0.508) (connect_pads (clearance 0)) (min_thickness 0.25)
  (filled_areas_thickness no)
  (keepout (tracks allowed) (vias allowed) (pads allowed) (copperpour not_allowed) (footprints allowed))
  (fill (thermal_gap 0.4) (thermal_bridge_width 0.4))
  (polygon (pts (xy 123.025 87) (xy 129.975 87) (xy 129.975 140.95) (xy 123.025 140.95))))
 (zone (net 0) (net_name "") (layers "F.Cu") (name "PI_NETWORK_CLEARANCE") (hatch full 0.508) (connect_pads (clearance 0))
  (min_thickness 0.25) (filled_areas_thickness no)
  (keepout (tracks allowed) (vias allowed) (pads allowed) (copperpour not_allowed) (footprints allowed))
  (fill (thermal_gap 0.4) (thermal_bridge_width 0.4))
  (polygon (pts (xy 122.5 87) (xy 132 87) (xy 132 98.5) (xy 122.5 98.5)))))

